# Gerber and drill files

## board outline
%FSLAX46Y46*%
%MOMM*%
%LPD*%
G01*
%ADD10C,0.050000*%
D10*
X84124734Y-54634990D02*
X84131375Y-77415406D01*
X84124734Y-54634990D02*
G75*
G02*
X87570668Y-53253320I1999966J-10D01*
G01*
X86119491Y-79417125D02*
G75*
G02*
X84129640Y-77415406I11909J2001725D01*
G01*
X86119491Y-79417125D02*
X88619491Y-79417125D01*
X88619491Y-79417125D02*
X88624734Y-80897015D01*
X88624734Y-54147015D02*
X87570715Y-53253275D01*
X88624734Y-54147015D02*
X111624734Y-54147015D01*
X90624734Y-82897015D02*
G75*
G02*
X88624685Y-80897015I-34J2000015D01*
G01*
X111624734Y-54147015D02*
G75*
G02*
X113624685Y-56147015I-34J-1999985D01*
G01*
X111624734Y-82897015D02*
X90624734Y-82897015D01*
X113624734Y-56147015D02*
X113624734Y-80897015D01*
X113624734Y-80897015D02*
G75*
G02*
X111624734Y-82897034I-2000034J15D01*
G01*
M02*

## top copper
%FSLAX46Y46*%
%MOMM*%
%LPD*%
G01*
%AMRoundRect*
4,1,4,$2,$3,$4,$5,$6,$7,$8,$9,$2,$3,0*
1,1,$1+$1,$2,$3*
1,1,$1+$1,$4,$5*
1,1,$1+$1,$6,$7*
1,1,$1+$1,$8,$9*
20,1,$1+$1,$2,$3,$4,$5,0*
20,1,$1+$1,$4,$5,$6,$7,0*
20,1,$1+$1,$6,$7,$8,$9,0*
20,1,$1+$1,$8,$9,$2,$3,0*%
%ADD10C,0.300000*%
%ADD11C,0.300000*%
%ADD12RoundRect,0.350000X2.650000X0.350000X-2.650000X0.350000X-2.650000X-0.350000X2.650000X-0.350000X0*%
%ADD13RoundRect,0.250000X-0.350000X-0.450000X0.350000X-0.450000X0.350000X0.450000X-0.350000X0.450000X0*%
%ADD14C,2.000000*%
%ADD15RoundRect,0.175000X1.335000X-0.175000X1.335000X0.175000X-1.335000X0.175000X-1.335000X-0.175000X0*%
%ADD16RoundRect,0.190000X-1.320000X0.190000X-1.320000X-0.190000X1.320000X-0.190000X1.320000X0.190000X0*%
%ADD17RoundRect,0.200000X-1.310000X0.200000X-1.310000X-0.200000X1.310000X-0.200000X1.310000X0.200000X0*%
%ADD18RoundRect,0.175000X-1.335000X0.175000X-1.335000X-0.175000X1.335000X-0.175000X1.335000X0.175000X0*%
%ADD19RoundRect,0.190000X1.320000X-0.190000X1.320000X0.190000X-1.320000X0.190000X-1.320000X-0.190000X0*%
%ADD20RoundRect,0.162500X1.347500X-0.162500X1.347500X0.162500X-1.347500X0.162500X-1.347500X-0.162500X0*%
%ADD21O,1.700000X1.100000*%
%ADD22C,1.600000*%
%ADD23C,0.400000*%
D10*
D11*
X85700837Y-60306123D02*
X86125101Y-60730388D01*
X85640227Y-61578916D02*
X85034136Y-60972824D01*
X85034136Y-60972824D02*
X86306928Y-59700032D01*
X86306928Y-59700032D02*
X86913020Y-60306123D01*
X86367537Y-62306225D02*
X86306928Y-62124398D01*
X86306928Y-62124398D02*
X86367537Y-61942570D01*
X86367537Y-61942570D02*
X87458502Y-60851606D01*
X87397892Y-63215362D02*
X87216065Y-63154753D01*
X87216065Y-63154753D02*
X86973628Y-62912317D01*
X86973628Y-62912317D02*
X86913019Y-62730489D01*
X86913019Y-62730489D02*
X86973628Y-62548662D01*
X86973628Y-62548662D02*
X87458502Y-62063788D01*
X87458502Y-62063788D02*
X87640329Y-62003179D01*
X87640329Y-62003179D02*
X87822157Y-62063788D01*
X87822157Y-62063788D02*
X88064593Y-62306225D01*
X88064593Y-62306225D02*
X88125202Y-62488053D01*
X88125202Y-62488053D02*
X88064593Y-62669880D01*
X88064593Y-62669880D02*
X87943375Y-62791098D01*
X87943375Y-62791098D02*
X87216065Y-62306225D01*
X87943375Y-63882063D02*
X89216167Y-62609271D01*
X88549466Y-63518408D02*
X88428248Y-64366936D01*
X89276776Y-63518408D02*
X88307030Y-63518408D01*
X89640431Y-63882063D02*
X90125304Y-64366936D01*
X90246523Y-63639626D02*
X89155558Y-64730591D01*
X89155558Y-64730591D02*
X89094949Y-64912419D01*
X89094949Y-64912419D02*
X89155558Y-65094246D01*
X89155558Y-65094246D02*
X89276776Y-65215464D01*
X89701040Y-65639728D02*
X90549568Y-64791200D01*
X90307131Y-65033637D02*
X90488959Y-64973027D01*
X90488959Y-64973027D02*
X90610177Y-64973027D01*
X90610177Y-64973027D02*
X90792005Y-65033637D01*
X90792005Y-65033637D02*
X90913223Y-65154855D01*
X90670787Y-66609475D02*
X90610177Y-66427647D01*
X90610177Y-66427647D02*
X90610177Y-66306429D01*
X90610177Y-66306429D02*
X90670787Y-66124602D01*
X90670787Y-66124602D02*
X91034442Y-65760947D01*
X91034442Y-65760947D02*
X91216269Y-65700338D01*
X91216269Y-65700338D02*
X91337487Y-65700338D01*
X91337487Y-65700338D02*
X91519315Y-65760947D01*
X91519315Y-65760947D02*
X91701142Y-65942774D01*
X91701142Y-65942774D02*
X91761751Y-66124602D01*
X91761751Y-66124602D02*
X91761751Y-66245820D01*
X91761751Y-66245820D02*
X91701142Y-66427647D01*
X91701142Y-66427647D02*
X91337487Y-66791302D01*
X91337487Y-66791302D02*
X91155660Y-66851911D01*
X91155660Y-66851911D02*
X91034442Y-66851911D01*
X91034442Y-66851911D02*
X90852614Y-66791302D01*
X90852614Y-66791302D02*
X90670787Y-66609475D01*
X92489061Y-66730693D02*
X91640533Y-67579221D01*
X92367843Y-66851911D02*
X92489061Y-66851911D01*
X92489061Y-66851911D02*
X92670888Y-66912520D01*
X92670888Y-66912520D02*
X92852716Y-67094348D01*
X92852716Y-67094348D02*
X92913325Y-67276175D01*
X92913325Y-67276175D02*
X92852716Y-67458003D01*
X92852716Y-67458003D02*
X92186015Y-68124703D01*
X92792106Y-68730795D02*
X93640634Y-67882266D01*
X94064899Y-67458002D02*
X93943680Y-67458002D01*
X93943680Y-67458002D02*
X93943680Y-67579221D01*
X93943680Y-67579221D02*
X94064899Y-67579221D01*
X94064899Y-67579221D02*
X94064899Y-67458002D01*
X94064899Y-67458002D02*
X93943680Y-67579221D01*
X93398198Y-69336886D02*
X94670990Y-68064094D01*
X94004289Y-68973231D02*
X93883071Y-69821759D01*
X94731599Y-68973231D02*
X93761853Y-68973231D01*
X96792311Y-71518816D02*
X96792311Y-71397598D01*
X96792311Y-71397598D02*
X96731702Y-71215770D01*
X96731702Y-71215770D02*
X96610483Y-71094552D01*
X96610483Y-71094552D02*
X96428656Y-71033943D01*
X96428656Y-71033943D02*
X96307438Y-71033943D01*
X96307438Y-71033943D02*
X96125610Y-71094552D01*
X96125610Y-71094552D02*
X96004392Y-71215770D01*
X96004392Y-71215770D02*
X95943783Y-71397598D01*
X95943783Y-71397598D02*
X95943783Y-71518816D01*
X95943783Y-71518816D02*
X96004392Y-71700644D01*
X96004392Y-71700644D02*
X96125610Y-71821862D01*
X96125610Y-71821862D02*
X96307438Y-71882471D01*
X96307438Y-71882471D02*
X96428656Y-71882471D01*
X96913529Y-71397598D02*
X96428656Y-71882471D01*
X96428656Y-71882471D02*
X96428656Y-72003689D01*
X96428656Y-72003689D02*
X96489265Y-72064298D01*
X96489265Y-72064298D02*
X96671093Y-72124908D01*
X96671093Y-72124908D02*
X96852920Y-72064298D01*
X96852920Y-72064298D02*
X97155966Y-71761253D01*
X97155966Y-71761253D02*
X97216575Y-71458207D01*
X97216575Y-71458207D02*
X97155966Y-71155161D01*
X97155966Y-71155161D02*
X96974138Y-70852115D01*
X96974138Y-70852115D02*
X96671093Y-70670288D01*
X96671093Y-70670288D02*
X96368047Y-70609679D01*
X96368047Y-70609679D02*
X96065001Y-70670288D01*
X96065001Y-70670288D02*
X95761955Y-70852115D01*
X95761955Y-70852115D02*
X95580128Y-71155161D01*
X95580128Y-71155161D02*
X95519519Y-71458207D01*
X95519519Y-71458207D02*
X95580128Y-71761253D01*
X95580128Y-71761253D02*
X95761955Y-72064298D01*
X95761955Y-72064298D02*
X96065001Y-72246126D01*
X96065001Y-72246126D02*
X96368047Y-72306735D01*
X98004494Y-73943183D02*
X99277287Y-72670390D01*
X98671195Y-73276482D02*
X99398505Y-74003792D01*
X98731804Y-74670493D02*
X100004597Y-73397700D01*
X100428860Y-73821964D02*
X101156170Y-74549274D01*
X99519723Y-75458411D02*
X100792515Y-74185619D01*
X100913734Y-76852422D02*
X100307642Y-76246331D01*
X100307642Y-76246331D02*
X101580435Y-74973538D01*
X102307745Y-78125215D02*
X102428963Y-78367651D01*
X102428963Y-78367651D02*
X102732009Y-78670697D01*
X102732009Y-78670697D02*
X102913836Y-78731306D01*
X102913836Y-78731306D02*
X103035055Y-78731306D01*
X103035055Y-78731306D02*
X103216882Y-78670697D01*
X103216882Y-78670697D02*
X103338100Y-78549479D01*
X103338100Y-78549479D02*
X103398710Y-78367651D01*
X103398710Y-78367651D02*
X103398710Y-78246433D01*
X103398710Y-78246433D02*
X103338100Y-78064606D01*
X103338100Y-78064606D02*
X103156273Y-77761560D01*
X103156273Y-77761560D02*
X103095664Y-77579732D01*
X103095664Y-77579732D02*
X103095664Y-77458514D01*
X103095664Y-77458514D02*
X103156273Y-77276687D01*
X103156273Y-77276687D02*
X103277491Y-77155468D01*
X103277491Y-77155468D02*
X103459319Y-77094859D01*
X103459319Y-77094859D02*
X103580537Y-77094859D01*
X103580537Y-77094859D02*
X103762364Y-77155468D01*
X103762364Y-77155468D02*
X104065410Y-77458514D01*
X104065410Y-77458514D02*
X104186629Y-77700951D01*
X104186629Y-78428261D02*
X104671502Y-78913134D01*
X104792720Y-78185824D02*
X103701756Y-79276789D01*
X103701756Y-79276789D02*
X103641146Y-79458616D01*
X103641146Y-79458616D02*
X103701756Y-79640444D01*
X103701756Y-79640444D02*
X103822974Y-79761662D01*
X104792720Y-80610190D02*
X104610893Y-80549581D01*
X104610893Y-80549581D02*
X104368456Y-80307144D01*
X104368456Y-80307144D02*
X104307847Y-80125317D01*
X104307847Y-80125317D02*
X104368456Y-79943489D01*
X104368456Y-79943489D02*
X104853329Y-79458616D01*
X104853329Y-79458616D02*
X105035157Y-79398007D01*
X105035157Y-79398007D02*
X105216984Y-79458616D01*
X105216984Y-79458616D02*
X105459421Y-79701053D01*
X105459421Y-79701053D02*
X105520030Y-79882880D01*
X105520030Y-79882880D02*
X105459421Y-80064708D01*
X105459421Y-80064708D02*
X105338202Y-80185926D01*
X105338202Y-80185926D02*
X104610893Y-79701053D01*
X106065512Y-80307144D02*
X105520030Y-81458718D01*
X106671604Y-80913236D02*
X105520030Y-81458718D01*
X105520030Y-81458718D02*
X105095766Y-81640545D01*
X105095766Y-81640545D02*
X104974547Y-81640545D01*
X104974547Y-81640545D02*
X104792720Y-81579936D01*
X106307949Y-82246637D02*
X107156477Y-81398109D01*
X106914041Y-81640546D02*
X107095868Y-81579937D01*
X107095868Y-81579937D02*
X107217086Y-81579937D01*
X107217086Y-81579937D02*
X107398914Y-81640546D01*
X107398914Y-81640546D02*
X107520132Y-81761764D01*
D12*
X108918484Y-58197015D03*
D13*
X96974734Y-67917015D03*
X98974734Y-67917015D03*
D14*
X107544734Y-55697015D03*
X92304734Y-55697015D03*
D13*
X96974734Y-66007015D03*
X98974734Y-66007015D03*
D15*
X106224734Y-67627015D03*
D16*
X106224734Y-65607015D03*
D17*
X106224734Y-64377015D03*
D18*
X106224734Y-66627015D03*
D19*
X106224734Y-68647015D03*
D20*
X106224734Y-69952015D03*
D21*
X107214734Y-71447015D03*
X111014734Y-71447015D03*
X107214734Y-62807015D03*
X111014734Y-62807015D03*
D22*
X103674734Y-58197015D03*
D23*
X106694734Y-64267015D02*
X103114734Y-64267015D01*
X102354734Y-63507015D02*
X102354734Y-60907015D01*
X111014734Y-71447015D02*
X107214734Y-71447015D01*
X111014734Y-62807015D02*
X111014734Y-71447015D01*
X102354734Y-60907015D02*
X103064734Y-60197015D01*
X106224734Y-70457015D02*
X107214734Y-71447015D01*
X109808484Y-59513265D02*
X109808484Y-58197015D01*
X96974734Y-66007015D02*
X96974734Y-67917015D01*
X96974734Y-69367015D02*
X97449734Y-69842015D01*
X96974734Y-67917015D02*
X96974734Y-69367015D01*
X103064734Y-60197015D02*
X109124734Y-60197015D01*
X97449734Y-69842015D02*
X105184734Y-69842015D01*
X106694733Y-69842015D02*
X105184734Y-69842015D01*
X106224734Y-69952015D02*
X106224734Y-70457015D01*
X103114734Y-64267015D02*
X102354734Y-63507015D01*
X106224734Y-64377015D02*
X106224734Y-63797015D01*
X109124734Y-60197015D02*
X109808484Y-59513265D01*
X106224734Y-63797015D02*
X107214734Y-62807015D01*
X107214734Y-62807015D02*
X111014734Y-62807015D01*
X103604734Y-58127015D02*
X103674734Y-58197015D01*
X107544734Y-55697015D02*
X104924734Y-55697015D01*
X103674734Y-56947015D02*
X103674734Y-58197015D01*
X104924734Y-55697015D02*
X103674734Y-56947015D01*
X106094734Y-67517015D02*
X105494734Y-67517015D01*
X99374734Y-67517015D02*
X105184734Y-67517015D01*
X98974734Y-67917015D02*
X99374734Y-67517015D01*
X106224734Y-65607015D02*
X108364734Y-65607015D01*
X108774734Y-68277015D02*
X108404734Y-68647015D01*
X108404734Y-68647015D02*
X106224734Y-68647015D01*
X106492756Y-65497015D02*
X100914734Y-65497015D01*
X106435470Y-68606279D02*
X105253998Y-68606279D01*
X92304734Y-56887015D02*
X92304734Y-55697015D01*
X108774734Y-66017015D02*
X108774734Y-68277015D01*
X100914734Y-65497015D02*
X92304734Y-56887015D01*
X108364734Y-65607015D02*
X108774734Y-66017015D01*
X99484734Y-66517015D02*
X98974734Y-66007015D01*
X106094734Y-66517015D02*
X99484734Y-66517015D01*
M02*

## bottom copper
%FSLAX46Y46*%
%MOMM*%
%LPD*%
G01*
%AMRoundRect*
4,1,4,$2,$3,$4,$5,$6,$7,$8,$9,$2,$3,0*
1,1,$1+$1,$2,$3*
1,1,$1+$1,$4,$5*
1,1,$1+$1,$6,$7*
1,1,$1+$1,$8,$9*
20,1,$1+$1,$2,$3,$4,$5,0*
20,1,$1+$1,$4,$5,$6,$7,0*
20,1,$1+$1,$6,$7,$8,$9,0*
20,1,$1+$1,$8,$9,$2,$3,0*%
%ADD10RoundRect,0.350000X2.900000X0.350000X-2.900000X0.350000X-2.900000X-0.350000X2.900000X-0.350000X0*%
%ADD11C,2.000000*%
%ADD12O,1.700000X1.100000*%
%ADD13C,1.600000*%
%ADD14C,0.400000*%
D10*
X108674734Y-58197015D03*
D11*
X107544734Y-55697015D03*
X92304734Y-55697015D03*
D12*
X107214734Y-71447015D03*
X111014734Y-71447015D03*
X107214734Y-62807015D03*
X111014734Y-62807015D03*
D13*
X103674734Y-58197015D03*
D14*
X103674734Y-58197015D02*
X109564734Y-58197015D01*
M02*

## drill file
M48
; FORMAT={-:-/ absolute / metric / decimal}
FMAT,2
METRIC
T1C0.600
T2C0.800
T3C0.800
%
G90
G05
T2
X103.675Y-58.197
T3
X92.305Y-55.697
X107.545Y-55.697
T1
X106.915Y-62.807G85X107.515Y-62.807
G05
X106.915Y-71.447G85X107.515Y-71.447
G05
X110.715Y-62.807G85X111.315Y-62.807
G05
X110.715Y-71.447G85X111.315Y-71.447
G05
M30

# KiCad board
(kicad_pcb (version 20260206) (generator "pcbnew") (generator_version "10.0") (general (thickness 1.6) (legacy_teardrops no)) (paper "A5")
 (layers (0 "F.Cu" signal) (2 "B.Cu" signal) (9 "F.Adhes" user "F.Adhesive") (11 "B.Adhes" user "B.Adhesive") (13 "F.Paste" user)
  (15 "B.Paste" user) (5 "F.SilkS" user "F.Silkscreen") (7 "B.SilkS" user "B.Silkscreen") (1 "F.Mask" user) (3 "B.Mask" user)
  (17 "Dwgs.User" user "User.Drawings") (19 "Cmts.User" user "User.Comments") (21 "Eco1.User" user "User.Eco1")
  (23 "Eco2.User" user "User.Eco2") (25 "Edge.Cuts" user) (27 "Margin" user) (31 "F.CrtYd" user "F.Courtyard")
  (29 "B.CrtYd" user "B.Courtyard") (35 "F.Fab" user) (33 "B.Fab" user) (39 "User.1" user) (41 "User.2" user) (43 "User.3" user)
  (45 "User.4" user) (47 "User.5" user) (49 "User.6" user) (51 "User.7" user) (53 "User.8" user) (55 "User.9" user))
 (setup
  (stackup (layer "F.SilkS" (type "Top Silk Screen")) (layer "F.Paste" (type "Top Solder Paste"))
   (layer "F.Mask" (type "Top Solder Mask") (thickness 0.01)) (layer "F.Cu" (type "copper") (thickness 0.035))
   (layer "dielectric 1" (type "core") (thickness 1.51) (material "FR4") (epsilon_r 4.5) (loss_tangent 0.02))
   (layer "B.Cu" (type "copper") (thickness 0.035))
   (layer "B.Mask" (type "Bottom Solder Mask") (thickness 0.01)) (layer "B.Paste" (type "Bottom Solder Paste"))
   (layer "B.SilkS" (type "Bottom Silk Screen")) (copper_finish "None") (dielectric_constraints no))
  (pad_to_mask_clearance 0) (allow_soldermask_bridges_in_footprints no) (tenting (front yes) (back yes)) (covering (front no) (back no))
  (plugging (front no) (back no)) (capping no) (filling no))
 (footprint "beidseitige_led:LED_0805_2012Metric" (layer "F.Cu") (at 110.424734 58.197015 180)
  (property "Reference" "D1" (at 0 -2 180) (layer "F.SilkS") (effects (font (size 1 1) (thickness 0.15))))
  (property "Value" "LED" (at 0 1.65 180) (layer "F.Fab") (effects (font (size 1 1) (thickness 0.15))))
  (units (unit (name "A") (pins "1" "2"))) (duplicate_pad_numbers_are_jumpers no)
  (pad "1" smd roundrect (at 1.50625 0 180) (size 6 1.4) (layers "F.Cu" "F.Mask" "F.Paste") (roundrect_rratio 0.25) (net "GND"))
  (pad "2" smd roundrect (at 1.75 0 180) (size 6.5 1.4) (layers "B.Cu" "B.Mask" "B.Paste") (roundrect_rratio 0.25) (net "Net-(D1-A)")))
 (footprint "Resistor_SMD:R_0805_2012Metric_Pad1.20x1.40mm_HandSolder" (layer "F.Cu") (at 97.974734 67.917015)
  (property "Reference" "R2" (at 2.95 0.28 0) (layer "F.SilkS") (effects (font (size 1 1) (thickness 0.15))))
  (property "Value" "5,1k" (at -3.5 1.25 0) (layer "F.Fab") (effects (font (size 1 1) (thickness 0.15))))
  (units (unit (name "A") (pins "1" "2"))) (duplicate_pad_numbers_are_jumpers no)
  (pad "1" smd roundrect (at -1 0) (size 1.2 1.4) (layers "F.Cu" "F.Mask" "F.Paste") (roundrect_rratio 0.208333) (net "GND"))
  (pad "2" smd roundrect (at 1 0) (size 1.2 1.4) (layers "F.Cu" "F.Mask" "F.Paste") (roundrect_rratio 0.208333) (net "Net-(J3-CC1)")))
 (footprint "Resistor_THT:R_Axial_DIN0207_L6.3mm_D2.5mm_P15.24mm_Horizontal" (layer "F.Cu") (at 107.544734 55.697015 180)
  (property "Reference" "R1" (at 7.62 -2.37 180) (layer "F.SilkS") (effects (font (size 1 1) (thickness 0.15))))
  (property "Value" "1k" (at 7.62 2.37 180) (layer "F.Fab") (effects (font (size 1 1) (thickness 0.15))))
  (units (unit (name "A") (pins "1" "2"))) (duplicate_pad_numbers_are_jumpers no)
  (pad "1" thru_hole circle (at 0 0 180) (size 2 2) (drill 0.8) (layers "*.Cu" "*.Mask") (remove_unused_layers no) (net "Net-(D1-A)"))
  (pad "2" thru_hole circle (at 15.24 0 180) (size 2 2) (drill 0.8) (layers "*.Cu" "*.Mask") (remove_unused_layers no) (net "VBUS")))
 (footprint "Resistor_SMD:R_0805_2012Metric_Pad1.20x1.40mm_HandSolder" (layer "F.Cu") (at 97.974734 66.007015)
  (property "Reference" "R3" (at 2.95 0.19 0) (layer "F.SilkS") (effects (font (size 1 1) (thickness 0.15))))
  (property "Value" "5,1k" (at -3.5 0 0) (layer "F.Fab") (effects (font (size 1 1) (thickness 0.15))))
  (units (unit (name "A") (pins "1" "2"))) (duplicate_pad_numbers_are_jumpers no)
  (pad "1" smd roundrect (at -1 0) (size 1.2 1.4) (layers "F.Cu" "F.Mask" "F.Paste") (roundrect_rratio 0.208333) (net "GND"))
  (pad "2" smd roundrect (at 1 0) (size 1.2 1.4) (layers "F.Cu" "F.Mask" "F.Paste") (roundrect_rratio 0.208333) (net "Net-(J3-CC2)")))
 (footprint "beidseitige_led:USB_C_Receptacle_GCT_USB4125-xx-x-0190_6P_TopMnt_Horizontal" (layer "F.Cu") (at 110.214734 67.127015 90)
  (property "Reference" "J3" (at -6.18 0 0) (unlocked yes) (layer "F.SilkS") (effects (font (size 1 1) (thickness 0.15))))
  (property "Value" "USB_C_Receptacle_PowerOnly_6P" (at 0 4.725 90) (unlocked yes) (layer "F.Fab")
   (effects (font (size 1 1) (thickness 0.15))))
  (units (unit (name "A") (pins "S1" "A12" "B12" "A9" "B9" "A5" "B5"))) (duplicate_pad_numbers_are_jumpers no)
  (pad "A5" smd roundrect (at -0.5 -3.99 90) (size 0.7 3.02) (layers "F.Cu" "F.Mask" "F.Paste") (roundrect_rratio 0.25) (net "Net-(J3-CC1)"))
  (pad "A9" smd roundrect (at 1.52 -3.99 270) (size 0.76 3.02) (layers "F.Cu" "F.Mask" "F.Paste") (roundrect_rratio 0.25) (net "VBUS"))
  (pad "A12" smd roundrect (at 2.75 -3.99 270) (size 0.8 3.02) (layers "F.Cu" "F.Mask" "F.Paste") (roundrect_rratio 0.25) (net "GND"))
  (pad "B5" smd roundrect (at 0.5 -3.99 270) (size 0.7 3.02) (layers "F.Cu" "F.Mask" "F.Paste") (roundrect_rratio 0.25) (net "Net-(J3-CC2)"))
  (pad "B9" smd roundrect (at -1.52 -3.99 90) (size 0.76 3.02) (layers "F.Cu" "F.Mask" "F.Paste") (roundrect_rratio 0.25) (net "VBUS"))
  (pad "B12" smd roundrect (at -2.825 -3.99 90) (size 0.65 3.02) (layers "F.Cu" "F.Mask" "F.Paste") (roundrect_rratio 0.25) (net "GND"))
  (pad "S1" thru_hole oval (at -4.32 -3 90) (size 1.1 1.7) (drill oval 0.6 1.2) (layers "*.Cu" "*.Mask" "F.Paste") (remove_unused_layers no)
   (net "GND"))
  (pad "S1" thru_hole oval (at -4.32 0.8 90) (size 1.1 1.7) (drill oval 0.6 1.2) (layers "*.Cu" "*.Mask" "F.Paste")
   (remove_unused_layers no) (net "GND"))
  (pad "S1" thru_hole oval (at 4.32 -3 90) (size 1.1 1.7) (drill oval 0.6 1.2) (layers "*.Cu" "*.Mask" "F.Paste") (remove_unused_layers no)
   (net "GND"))
  (pad "S1" thru_hole oval (at 4.32 0.8 90) (size 1.1 1.7) (drill oval 0.6 1.2) (layers "*.Cu" "*.Mask" "F.Paste") (remove_unused_layers no)
   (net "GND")))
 (gr_line (start 84.124734 54.63499) (end 84.131375 77.415406) (stroke (width 0.05) (type default)) (layer "Edge.Cuts"))
 (gr_arc (start 84.124734 54.63499) (mid 85.380413 52.778678) (end 87.570715 53.253275) (stroke (width 0.05) (type default))
  (layer "Edge.Cuts"))
 (gr_arc (start 86.119491 79.417125) (mid 84.711734 78.826646) (end 84.129621 77.415406) (stroke (width 0.05) (type default))
  (layer "Edge.Cuts"))
 (gr_line (start 86.119491 79.417125) (end 88.619491 79.417125) (stroke (width 0.05) (type default)) (layer "Edge.Cuts"))
 (gr_line (start 88.619491 79.417125) (end 88.624734 80.897015) (stroke (width 0.05) (type default)) (layer "Edge.Cuts"))
 (gr_line (start 88.624734 54.147015) (end 87.570715 53.253275) (stroke (width 0.05) (type default)) (layer "Edge.Cuts"))
 (gr_line (start 88.624734 54.147015) (end 111.624734 54.147015) (stroke (width 0.05) (type default)) (layer "Edge.Cuts"))
 (gr_arc (start 90.624734 82.897015) (mid 89.21052 82.311229) (end 88.624734 80.897015) (stroke (width 0.05) (type default))
  (layer "Edge.Cuts"))
 (gr_arc (start 111.624734 54.147015) (mid 113.038948 54.732801) (end 113.624734 56.147015) (stroke (width 0.05) (type default))
  (layer "Edge.Cuts"))
 (gr_line (start 111.624734 82.897015) (end 90.624734 82.897015) (stroke (width 0.05) (type default)) (layer "Edge.Cuts"))
 (gr_line (start 113.624734 56.147015) (end 113.624734 80.897015) (stroke (width 0.05) (type default)) (layer "Edge.Cuts"))
 (gr_arc (start 113.624734 80.897015) (mid 113.038948 82.311229) (end 111.624734 82.897015) (stroke (width 0.05) (type default))
  (layer "Edge.Cuts"))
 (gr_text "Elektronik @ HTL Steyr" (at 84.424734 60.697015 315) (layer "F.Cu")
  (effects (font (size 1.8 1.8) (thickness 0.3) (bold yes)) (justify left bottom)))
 (segment (start 106.694734 64.267015) (end 103.114734 64.267015) (width 0.4) (layer "F.Cu") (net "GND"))
 (segment (start 102.354734 63.507015) (end 102.354734 60.907015) (width 0.4) (layer "F.Cu") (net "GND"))
 (segment (start 111.014734 71.447015) (end 107.214734 71.447015) (width 0.4) (layer "F.Cu") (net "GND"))
 (segment (start 111.014734 62.807015) (end 111.014734 71.447015) (width 0.4) (layer "F.Cu") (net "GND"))
 (segment (start 102.354734 60.907015) (end 103.064734 60.197015) (width 0.4) (layer "F.Cu") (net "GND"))
 (segment (start 106.224734 70.457015) (end 107.214734 71.447015) (width 0.4) (layer "F.Cu") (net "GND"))
 (segment (start 109.808484 59.513265) (end 109.808484 58.197015) (width 0.4) (layer "F.Cu") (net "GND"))
 (segment (start 96.974734 66.007015) (end 96.974734 67.917015) (width 0.4) (layer "F.Cu") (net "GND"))
 (segment (start 96.974734 69.367015) (end 97.449734 69.842015) (width 0.4) (layer "F.Cu") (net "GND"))
 (segment (start 96.974734 67.917015) (end 96.974734 69.367015) (width 0.4) (layer "F.Cu") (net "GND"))
 (segment (start 103.064734 60.197015) (end 109.124734 60.197015) (width 0.4) (layer "F.Cu") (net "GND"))
 (segment (start 97.449734 69.842015) (end 105.184734 69.842015) (width 0.4) (layer "F.Cu") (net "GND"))
 (segment (start 106.694733 69.842015) (end 105.184734 69.842015) (width 0.4) (layer "F.Cu") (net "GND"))
 (segment (start 106.224734 69.952015) (end 106.224734 70.457015) (width 0.4) (layer "F.Cu") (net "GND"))
 (segment (start 103.114734 64.267015) (end 102.354734 63.507015) (width 0.4) (layer "F.Cu") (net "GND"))
 (segment (start 106.224734 64.377015) (end 106.224734 63.797015) (width 0.4) (layer "F.Cu") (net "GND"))
 (segment (start 109.124734 60.197015) (end 109.808484 59.513265) (width 0.4) (layer "F.Cu") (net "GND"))
 (segment (start 106.224734 63.797015) (end 107.214734 62.807015) (width 0.4) (layer "F.Cu") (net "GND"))
 (segment (start 107.214734 62.807015) (end 111.014734 62.807015) (width 0.4) (layer "F.Cu") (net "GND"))
 (segment (start 103.604734 58.127015) (end 103.674734 58.197015) (width 0.4) (layer "F.Cu") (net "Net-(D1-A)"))
 (segment (start 107.544734 55.697015) (end 104.924734 55.697015) (width 0.4) (layer "F.Cu") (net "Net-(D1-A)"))
 (segment (start 103.674734 56.947015) (end 103.674734 58.197015) (width 0.4) (layer "F.Cu") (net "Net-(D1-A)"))
 (segment (start 104.924734 55.697015) (end 103.674734 56.947015) (width 0.4) (layer "F.Cu") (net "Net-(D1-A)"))
 (via (at 103.674734 58.197015) (size 1.6) (drill 0.8) (layers "F.Cu" "B.Cu") (capping no) (covering (front no) (back no))
  (plugging (front no) (back no)) (filling no) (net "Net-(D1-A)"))
 (segment (start 103.674734 58.197015) (end 109.564734 58.197015) (width 0.4) (layer "B.Cu") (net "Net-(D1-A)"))
 (segment (start 106.094734 67.517015) (end 105.494734 67.517015) (width 0.4) (layer "F.Cu") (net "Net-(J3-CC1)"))
 (segment (start 99.374734 67.517015) (end 105.184734 67.517015) (width 0.4) (layer "F.Cu") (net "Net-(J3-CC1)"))
 (segment (start 98.974734 67.917015) (end 99.374734 67.517015) (width 0.4) (layer "F.Cu") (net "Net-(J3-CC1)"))
 (segment (start 106.224734 65.607015) (end 108.364734 65.607015) (width 0.4) (layer "F.Cu") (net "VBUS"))
 (segment (start 108.774734 68.277015) (end 108.404734 68.647015) (width 0.4) (layer "F.Cu") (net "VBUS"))
 (segment (start 108.404734 68.647015) (end 106.224734 68.647015) (width 0.4) (layer "F.Cu") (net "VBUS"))
 (segment (start 106.492756 65.497015) (end 100.914734 65.497015) (width 0.4) (layer "F.Cu") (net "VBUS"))
 (segment (start 106.43547 68.606279) (end 105.253998 68.606279) (width 0.4) (layer "F.Cu") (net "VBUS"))
 (segment (start 92.304734 56.887015) (end 92.304734 55.697015) (width 0.4) (layer "F.Cu") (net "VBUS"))
 (segment (start 108.774734 66.017015) (end 108.774734 68.277015) (width 0.4) (layer "F.Cu") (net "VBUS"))
 (segment (start 100.914734 65.497015) (end 92.304734 56.887015) (width 0.4) (layer "F.Cu") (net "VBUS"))
 (segment (start 108.364734 65.607015) (end 108.774734 66.017015) (width 0.4) (layer "F.Cu") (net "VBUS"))
 (segment (start 99.484734 66.517015) (end 98.974734 66.007015) (width 0.4) (layer "F.Cu") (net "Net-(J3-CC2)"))
 (segment (start 106.094734 66.517015) (end 99.484734 66.517015) (width 0.4) (layer "F.Cu") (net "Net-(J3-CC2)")))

